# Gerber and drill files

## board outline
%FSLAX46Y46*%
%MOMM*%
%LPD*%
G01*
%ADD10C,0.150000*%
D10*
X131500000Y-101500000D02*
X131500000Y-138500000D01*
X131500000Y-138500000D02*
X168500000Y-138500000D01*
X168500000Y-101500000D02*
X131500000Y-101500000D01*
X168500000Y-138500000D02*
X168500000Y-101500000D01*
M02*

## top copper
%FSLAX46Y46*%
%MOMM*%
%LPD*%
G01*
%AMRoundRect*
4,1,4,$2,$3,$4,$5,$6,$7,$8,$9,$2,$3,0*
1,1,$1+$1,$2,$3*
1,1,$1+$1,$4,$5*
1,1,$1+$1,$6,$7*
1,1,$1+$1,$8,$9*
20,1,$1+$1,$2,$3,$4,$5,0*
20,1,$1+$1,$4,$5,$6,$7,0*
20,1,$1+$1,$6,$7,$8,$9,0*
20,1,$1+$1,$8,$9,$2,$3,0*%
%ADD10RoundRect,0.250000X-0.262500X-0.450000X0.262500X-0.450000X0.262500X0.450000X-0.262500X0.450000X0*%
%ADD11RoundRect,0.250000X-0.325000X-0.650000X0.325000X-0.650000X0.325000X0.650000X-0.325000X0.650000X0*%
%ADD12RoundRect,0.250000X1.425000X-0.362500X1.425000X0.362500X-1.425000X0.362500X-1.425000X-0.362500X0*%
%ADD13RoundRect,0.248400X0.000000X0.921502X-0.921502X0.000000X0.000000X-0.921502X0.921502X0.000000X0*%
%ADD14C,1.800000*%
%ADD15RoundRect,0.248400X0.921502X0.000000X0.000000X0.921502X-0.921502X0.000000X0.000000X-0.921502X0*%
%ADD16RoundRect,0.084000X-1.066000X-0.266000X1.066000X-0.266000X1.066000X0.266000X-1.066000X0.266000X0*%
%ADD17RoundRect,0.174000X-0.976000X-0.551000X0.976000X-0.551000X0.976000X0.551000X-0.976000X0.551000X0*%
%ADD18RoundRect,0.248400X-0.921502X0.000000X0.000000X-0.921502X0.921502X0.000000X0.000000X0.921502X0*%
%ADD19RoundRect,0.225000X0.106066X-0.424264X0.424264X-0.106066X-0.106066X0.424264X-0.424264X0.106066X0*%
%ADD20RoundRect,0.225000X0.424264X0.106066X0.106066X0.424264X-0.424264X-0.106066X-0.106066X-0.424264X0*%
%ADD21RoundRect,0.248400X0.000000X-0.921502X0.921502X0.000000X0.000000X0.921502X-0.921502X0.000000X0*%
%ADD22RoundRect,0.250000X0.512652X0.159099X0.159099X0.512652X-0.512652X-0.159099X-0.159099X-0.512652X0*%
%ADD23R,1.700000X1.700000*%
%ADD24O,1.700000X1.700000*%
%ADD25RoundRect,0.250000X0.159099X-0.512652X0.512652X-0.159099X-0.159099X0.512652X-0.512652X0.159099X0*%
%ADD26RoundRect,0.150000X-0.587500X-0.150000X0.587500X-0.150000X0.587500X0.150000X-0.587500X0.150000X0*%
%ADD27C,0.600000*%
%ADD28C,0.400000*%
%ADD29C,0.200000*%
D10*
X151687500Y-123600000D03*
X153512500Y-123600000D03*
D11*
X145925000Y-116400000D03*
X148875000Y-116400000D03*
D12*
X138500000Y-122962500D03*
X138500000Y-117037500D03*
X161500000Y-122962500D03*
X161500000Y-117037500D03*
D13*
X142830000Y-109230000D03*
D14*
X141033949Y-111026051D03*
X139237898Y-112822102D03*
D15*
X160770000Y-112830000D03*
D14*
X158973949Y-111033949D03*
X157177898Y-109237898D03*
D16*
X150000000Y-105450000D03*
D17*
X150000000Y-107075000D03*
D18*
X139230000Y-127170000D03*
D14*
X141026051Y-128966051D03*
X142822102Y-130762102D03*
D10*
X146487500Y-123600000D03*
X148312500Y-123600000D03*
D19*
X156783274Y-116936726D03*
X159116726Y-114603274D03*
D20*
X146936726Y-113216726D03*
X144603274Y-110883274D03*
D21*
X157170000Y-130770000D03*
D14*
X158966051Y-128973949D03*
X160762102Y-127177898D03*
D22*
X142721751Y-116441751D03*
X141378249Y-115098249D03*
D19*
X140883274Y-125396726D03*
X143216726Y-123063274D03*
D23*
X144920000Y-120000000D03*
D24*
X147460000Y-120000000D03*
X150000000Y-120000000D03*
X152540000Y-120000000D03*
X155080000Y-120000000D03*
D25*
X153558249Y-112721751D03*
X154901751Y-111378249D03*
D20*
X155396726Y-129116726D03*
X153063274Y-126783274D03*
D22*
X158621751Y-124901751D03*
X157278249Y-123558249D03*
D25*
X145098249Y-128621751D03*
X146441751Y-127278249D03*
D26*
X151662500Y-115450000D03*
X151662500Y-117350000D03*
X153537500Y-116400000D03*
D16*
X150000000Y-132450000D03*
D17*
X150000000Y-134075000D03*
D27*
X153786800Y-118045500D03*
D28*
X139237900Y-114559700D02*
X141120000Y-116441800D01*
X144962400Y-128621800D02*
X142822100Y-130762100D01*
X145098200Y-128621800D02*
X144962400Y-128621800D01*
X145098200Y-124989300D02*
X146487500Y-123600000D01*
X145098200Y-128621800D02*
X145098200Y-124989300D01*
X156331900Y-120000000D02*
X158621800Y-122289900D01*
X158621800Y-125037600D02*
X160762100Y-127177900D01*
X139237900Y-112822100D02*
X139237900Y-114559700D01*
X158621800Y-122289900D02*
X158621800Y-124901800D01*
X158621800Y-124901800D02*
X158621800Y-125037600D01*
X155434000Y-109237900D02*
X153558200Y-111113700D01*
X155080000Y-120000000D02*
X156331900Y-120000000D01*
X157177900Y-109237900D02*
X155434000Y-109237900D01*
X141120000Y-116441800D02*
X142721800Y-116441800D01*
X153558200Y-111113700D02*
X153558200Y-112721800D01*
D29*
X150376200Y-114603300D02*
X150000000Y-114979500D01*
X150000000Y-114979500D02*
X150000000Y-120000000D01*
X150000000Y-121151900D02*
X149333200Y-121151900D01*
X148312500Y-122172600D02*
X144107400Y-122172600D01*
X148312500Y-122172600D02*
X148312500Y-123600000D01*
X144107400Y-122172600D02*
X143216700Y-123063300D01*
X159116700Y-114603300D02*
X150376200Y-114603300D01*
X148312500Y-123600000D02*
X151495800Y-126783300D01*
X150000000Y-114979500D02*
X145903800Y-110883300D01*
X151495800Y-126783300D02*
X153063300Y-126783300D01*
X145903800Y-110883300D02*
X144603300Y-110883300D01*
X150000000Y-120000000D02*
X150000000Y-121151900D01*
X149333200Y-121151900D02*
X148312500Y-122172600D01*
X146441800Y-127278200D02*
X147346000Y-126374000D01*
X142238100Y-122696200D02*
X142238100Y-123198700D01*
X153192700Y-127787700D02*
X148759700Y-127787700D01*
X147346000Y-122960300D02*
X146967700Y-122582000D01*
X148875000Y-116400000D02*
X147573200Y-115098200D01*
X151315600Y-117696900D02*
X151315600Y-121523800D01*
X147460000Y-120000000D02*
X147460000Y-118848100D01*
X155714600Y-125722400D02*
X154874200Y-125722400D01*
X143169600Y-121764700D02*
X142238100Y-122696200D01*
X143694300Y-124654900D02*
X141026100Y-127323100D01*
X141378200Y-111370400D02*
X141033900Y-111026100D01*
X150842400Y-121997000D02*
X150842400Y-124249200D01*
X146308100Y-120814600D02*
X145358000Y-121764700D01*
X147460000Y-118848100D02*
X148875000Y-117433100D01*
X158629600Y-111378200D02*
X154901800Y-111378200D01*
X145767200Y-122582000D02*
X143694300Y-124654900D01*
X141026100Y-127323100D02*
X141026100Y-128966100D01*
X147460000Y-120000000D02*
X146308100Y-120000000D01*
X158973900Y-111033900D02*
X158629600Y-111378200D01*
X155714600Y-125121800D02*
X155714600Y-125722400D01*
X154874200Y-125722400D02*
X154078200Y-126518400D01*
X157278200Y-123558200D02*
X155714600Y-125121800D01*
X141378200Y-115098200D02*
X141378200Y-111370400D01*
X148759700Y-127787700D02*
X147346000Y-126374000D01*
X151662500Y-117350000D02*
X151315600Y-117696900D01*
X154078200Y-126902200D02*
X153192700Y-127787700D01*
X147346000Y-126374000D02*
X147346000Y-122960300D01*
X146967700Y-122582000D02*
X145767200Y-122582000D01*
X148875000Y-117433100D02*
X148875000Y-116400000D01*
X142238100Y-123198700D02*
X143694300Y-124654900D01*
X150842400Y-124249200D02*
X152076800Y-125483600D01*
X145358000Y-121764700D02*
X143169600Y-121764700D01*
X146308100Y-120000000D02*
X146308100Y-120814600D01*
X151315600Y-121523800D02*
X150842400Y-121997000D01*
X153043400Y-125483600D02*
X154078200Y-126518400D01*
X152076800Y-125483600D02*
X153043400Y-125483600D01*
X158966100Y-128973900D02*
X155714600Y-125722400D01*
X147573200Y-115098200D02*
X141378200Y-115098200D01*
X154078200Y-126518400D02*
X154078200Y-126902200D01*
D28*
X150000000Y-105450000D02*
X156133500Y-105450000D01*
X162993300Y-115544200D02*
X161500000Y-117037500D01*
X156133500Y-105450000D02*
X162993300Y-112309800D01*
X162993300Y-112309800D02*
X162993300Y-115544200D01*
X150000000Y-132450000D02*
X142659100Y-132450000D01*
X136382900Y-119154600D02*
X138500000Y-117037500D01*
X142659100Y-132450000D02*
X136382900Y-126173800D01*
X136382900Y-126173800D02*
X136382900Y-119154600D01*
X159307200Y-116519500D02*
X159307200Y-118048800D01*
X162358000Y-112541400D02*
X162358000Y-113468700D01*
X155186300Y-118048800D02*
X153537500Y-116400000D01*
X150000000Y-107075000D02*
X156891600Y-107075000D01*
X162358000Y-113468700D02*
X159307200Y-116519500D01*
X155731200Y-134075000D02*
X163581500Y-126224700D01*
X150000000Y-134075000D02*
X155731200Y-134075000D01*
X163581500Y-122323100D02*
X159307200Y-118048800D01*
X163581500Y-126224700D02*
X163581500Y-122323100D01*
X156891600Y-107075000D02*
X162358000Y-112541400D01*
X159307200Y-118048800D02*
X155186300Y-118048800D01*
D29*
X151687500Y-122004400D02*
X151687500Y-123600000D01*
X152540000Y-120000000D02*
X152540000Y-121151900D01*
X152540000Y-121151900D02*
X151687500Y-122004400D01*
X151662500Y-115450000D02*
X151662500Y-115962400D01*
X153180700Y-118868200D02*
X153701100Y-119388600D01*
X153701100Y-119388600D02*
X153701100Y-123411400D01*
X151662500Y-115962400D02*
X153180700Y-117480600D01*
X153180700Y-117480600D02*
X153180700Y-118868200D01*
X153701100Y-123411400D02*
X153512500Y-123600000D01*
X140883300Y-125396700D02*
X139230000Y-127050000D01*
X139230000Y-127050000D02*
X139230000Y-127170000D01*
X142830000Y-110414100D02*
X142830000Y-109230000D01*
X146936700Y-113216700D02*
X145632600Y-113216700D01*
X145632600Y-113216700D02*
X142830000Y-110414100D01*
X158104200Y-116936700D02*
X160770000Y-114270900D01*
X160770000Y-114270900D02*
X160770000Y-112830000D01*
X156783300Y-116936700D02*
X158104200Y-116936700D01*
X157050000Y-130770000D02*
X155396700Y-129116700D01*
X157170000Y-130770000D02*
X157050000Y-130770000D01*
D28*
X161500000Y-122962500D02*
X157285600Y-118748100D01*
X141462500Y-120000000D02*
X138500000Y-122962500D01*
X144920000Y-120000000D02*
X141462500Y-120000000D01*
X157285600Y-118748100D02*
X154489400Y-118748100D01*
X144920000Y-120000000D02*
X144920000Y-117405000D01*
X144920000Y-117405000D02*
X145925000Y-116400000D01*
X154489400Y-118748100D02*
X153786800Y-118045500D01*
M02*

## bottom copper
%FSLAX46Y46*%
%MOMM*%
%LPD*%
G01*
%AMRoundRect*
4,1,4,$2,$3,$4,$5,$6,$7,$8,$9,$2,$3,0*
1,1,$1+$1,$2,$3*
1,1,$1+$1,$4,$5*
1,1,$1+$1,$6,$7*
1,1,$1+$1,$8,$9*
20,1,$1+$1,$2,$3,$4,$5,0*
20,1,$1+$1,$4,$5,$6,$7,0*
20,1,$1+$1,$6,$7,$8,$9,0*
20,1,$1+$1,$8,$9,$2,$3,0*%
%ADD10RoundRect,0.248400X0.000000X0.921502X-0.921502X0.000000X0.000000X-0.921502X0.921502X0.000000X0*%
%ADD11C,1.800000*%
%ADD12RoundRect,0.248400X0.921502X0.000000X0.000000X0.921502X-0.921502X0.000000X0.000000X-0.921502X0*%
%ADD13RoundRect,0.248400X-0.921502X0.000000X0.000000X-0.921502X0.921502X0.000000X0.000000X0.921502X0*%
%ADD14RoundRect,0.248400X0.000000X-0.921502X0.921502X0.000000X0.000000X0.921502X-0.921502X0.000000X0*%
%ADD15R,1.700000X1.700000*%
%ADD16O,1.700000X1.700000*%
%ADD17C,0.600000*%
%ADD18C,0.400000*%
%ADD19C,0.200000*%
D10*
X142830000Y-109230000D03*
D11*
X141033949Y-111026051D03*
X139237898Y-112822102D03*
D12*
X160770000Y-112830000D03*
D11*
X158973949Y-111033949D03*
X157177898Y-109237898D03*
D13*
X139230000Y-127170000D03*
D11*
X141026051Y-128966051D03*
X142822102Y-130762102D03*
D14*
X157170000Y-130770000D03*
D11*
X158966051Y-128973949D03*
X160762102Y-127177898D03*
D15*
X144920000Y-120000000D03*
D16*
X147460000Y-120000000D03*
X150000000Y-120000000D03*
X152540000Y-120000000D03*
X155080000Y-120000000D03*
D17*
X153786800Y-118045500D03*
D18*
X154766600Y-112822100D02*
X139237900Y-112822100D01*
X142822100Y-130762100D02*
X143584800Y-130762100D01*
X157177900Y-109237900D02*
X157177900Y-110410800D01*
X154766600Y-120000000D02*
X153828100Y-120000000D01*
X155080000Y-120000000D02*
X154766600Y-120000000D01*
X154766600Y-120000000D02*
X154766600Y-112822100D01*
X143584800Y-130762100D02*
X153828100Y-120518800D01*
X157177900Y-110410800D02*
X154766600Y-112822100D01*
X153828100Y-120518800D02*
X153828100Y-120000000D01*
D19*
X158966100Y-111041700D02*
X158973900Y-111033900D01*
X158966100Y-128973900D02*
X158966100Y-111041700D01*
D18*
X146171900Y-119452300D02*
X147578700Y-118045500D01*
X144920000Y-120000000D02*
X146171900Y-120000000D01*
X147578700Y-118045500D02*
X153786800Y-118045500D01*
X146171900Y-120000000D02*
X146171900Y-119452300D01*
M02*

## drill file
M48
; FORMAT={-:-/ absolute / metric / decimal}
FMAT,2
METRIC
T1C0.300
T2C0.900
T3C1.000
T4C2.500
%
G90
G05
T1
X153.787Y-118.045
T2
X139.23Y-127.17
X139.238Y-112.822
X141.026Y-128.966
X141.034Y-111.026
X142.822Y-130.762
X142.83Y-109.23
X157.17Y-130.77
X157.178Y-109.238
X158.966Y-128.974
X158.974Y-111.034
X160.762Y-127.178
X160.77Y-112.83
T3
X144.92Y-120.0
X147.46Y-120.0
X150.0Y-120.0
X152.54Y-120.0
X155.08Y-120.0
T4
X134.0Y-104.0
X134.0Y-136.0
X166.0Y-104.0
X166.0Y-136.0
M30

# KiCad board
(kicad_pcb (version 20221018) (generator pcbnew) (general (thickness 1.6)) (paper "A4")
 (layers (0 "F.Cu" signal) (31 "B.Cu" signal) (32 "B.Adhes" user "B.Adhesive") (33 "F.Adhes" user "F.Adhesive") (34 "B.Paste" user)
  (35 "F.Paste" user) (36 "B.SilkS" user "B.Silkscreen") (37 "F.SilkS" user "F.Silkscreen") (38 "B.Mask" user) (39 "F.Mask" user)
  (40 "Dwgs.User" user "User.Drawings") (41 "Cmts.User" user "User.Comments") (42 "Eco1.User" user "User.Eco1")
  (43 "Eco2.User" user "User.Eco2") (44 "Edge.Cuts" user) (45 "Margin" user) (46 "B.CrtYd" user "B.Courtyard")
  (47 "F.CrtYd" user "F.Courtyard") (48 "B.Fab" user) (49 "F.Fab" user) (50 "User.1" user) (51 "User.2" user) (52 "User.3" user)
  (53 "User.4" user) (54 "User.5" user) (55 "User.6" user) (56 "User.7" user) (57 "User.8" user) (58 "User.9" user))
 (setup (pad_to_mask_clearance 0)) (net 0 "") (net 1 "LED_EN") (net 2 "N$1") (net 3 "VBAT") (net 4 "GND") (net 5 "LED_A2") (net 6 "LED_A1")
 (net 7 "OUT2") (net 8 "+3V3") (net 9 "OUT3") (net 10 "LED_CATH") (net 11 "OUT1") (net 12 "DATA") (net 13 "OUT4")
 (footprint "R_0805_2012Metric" (layer "F.Cu") (at 152.6 123.6)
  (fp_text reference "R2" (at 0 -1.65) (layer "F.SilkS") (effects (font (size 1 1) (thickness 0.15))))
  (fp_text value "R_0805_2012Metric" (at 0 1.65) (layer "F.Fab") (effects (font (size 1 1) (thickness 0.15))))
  (pad "1" smd roundrect (at -0.9125 0) (size 1.025 1.4) (layers "F.Cu" "F.Paste" "F.Mask") (roundrect_rratio 0.243902) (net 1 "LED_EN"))
  (pad "2" smd roundrect (at 0.9125 0) (size 1.025 1.4) (layers "F.Cu" "F.Paste" "F.Mask") (roundrect_rratio 0.243902) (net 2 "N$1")))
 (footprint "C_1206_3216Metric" (layer "F.Cu") (at 147.4 116.4)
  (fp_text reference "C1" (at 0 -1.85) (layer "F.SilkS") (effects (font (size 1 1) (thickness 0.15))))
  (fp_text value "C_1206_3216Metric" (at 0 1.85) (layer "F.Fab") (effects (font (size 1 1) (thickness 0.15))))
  (pad "1" smd roundrect (at -1.475 0) (size 1.15 1.8) (layers "F.Cu" "F.Paste" "F.Mask") (roundrect_rratio 0.217391) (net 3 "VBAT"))
  (pad "2" smd roundrect (at 1.475 0) (size 1.15 1.8) (layers "F.Cu" "F.Paste" "F.Mask") (roundrect_rratio 0.217391) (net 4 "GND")))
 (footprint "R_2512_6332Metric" (layer "F.Cu") (at 138.5 120 90)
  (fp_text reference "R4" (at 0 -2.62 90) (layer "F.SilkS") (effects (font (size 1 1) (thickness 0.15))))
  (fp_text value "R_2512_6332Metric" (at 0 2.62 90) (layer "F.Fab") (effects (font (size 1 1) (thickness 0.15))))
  (pad "1" smd roundrect (at -2.9625 0 90) (size 1.225 3.35) (layers "F.Cu" "F.Paste" "F.Mask") (roundrect_rratio 0.204082) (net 3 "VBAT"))
  (pad "2" smd roundrect (at 2.9625 0 90) (size 1.225 3.35) (layers "F.Cu" "F.Paste" "F.Mask") (roundrect_rratio 0.204082) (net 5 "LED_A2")))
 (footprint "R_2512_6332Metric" (layer "F.Cu") (at 161.5 120 90)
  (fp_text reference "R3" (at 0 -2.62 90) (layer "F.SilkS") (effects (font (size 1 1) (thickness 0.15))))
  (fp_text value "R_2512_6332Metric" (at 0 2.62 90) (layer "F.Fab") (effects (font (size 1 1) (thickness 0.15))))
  (pad "1" smd roundrect (at -2.9625 0 90) (size 1.225 3.35) (layers "F.Cu" "F.Paste" "F.Mask") (roundrect_rratio 0.204082) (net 3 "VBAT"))
  (pad "2" smd roundrect (at 2.9625 0 90) (size 1.225 3.35) (layers "F.Cu" "F.Paste" "F.Mask") (roundrect_rratio 0.204082) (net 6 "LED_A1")))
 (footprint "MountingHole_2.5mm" (layer "F.Cu") (at 134 104)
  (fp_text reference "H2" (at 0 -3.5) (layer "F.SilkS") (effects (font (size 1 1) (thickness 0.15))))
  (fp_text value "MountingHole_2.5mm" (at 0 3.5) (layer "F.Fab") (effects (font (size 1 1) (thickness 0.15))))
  (pad "" np_thru_hole circle (at 0 0) (size 2.5 2.5) (drill 2.5) (layers "*.Cu" "*.Mask")))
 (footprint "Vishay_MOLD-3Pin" (layer "F.Cu") (at 142.83 109.23 -135)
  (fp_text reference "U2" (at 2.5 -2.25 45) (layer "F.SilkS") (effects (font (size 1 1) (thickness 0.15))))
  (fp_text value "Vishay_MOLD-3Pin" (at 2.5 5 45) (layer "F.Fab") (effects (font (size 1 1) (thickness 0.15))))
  (pad "1" thru_hole roundrect (at 0 0 225) (size 1.8 1.8) (drill 0.9) (layers "*.Cu" "*.Mask") (roundrect_rratio 0.138) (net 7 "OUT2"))
  (pad "2" thru_hole circle (at 2.54 0 225) (size 1.8 1.8) (drill 0.9) (layers "*.Cu" "*.Mask") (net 4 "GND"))
  (pad "3" thru_hole circle (at 5.08 0 225) (size 1.8 1.8) (drill 0.9) (layers "*.Cu" "*.Mask") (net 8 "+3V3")))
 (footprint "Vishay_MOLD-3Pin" (layer "F.Cu") (at 160.77 112.83 135)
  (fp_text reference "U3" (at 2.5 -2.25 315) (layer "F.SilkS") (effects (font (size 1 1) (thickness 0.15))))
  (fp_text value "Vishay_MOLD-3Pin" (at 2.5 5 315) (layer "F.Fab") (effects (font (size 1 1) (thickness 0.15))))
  (pad "1" thru_hole roundrect (at 0 0 135) (size 1.8 1.8) (drill 0.9) (layers "*.Cu" "*.Mask") (roundrect_rratio 0.138) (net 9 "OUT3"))
  (pad "2" thru_hole circle (at 2.54 0 135) (size 1.8 1.8) (drill 0.9) (layers "*.Cu" "*.Mask") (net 4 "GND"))
  (pad "3" thru_hole circle (at 5.08 0 135) (size 1.8 1.8) (drill 0.9) (layers "*.Cu" "*.Mask") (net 8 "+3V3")))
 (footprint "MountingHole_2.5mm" (layer "F.Cu") (at 166 136)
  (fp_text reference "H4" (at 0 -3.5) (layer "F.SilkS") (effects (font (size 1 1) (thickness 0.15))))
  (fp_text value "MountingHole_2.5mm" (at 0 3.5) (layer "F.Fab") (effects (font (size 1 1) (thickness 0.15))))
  (pad "" np_thru_hole circle (at 0 0) (size 2.5 2.5) (drill 2.5) (layers "*.Cu" "*.Mask")))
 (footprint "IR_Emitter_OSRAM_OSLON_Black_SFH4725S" (layer "F.Cu") (at 150 106.5)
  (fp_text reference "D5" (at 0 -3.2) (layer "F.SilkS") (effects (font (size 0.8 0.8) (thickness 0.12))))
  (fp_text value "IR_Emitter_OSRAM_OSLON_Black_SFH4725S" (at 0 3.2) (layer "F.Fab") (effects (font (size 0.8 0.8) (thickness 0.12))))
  (pad "1" smd roundrect (at 0 -1.05) (size 2.3 0.7) (layers "F.Cu" "F.Paste" "F.Mask") (roundrect_rratio 0.12) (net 6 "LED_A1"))
  (pad "2" smd roundrect (at 0 0.575) (size 2.3 1.45) (layers "F.Cu" "F.Paste" "F.Mask") (roundrect_rratio 0.12) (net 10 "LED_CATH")))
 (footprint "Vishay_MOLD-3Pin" (layer "F.Cu") (at 139.23 127.17 -45)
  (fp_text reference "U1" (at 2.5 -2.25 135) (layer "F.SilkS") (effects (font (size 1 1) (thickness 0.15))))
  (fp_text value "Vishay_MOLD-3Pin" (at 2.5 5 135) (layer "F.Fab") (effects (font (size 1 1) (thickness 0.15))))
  (pad "1" thru_hole roundrect (at 0 0 315) (size 1.8 1.8) (drill 0.9) (layers "*.Cu" "*.Mask") (roundrect_rratio 0.138) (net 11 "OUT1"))
  (pad "2" thru_hole circle (at 2.54 0 315) (size 1.8 1.8) (drill 0.9) (layers "*.Cu" "*.Mask") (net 4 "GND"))
  (pad "3" thru_hole circle (at 5.08 0 315) (size 1.8 1.8) (drill 0.9) (layers "*.Cu" "*.Mask") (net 8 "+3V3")))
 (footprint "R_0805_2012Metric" (layer "F.Cu") (at 147.4 123.6)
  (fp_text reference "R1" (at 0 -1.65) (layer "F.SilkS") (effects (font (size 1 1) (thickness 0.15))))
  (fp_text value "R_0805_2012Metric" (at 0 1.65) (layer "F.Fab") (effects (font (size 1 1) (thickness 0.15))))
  (pad "1" smd roundrect (at -0.9125 0) (size 1.025 1.4) (layers "F.Cu" "F.Paste" "F.Mask") (roundrect_rratio 0.243902) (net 8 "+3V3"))
  (pad "2" smd roundrect (at 0.9125 0) (size 1.025 1.4) (layers "F.Cu" "F.Paste" "F.Mask") (roundrect_rratio 0.243902) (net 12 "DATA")))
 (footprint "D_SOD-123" (layer "F.Cu") (at 157.95 115.77 45)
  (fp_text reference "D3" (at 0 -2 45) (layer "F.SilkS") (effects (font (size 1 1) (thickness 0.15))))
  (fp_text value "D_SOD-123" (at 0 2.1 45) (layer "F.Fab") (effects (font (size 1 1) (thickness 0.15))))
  (pad "1" smd roundrect (at -1.65 0 45) (size 0.9 1.2) (layers "F.Cu" "F.Paste" "F.Mask") (roundrect_rratio 0.25) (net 9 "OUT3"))
  (pad "2" smd roundrect (at 1.65 0 45) (size 0.9 1.2) (layers "F.Cu" "F.Paste" "F.Mask") (roundrect_rratio 0.25) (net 12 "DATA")))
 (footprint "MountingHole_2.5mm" (layer "F.Cu") (at 134 136)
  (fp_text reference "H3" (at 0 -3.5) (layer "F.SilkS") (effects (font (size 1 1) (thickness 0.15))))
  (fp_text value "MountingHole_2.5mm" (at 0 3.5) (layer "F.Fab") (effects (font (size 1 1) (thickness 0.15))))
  (pad "" np_thru_hole circle (at 0 0) (size 2.5 2.5) (drill 2.5) (layers "*.Cu" "*.Mask")))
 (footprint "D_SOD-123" (layer "F.Cu") (at 145.77 112.05 135)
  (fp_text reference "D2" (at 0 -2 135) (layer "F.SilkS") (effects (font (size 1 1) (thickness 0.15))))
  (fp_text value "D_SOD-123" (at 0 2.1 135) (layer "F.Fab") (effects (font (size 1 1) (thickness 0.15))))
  (pad "1" smd roundrect (at -1.65 0 135) (size 0.9 1.2) (layers "F.Cu" "F.Paste" "F.Mask") (roundrect_rratio 0.25) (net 7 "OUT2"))
  (pad "2" smd roundrect (at 1.65 0 135) (size 0.9 1.2) (layers "F.Cu" "F.Paste" "F.Mask") (roundrect_rratio 0.25) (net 12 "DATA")))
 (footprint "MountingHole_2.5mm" (layer "F.Cu") (at 166 104)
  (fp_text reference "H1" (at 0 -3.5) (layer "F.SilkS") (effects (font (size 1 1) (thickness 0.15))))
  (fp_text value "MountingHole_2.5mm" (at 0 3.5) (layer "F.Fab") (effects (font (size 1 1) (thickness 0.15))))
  (pad "" np_thru_hole circle (at 0 0) (size 2.5 2.5) (drill 2.5) (layers "*.Cu" "*.Mask")))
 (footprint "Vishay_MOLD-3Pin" (layer "F.Cu") (at 157.17 130.77 45)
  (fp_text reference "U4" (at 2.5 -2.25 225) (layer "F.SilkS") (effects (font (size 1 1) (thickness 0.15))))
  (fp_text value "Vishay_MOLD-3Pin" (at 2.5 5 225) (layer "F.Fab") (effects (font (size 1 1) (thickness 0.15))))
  (pad "1" thru_hole roundrect (at 0 0 45) (size 1.8 1.8) (drill 0.9) (layers "*.Cu" "*.Mask") (roundrect_rratio 0.138) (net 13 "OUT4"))
  (pad "2" thru_hole circle (at 2.54 0 45) (size 1.8 1.8) (drill 0.9) (layers "*.Cu" "*.Mask") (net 4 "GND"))
  (pad "3" thru_hole circle (at 5.08 0 45) (size 1.8 1.8) (drill 0.9) (layers "*.Cu" "*.Mask") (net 8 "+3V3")))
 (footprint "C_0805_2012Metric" (layer "F.Cu") (at 142.05 115.77 135)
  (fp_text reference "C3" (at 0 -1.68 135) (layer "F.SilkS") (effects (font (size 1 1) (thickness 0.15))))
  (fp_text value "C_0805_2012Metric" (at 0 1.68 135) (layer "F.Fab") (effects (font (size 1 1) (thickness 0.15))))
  (pad "1" smd roundrect (at -0.95 0 135) (size 1 1.45) (layers "F.Cu" "F.Paste" "F.Mask") (roundrect_rratio 0.25) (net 8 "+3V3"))
  (pad "2" smd roundrect (at 0.95 0 135) (size 1 1.45) (layers "F.Cu" "F.Paste" "F.Mask") (roundrect_rratio 0.25) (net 4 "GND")))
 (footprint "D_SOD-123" (layer "F.Cu") (at 142.05 124.23 45)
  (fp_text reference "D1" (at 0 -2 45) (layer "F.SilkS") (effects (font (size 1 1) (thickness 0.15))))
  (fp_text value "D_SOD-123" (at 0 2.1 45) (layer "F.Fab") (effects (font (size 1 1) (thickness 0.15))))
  (pad "1" smd roundrect (at -1.65 0 45) (size 0.9 1.2) (layers "F.Cu" "F.Paste" "F.Mask") (roundrect_rratio 0.25) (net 11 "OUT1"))
  (pad "2" smd roundrect (at 1.65 0 45) (size 0.9 1.2) (layers "F.Cu" "F.Paste" "F.Mask") (roundrect_rratio 0.25) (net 12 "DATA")))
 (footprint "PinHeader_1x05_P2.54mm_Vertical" (layer "F.Cu") (at 144.92 120 90)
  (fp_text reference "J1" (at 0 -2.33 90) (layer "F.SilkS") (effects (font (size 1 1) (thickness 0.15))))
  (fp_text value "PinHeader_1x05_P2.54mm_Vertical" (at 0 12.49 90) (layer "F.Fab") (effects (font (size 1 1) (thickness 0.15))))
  (pad "1" thru_hole rect (at 0 0 90) (size 1.7 1.7) (drill 1) (layers "*.Cu" "*.Mask") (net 3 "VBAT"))
  (pad "2" thru_hole oval (at 0 2.54 90) (size 1.7 1.7) (drill 1) (layers "*.Cu" "*.Mask") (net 4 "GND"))
  (pad "3" thru_hole oval (at 0 5.08 90) (size 1.7 1.7) (drill 1) (layers "*.Cu" "*.Mask") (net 12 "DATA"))
  (pad "4" thru_hole oval (at 0 7.62 90) (size 1.7 1.7) (drill 1) (layers "*.Cu" "*.Mask") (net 1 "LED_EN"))
  (pad "5" thru_hole oval (at 0 10.16 90) (size 1.7 1.7) (drill 1) (layers "*.Cu" "*.Mask") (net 8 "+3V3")))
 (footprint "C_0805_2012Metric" (layer "F.Cu") (at 154.23 112.05 45)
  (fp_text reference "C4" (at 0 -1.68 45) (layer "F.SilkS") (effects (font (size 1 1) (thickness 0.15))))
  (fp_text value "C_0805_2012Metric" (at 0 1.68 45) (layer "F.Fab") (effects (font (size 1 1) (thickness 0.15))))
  (pad "1" smd roundrect (at -0.95 0 45) (size 1 1.45) (layers "F.Cu" "F.Paste" "F.Mask") (roundrect_rratio 0.25) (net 8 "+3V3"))
  (pad "2" smd roundrect (at 0.95 0 45) (size 1 1.45) (layers "F.Cu" "F.Paste" "F.Mask") (roundrect_rratio 0.25) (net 4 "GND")))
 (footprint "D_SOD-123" (layer "F.Cu") (at 154.23 127.95 135)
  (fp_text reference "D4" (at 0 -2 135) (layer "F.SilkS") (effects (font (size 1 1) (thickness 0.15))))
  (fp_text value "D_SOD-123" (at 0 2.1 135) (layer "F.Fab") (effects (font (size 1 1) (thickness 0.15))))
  (pad "1" smd roundrect (at -1.65 0 135) (size 0.9 1.2) (layers "F.Cu" "F.Paste" "F.Mask") (roundrect_rratio 0.25) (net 13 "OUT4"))
  (pad "2" smd roundrect (at 1.65 0 135) (size 0.9 1.2) (layers "F.Cu" "F.Paste" "F.Mask") (roundrect_rratio 0.25) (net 12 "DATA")))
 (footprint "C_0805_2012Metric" (layer "F.Cu") (at 157.95 124.23 135)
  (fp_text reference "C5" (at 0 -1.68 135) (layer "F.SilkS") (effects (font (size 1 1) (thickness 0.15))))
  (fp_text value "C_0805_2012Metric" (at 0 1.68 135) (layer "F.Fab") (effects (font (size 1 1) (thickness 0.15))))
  (pad "1" smd roundrect (at -0.95 0 135) (size 1 1.45) (layers "F.Cu" "F.Paste" "F.Mask") (roundrect_rratio 0.25) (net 8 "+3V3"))
  (pad "2" smd roundrect (at 0.95 0 135) (size 1 1.45) (layers "F.Cu" "F.Paste" "F.Mask") (roundrect_rratio 0.25) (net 4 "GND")))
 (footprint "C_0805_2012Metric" (layer "F.Cu") (at 145.77 127.95 45)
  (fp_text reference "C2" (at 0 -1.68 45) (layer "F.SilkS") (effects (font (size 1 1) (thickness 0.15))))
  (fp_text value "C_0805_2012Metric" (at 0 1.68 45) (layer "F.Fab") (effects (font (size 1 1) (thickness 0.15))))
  (pad "1" smd roundrect (at -0.95 0 45) (size 1 1.45) (layers "F.Cu" "F.Paste" "F.Mask") (roundrect_rratio 0.25) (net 8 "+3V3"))
  (pad "2" smd roundrect (at 0.95 0 45) (size 1 1.45) (layers "F.Cu" "F.Paste" "F.Mask") (roundrect_rratio 0.25) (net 4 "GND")))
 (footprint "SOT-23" (layer "F.Cu") (at 152.6 116.4)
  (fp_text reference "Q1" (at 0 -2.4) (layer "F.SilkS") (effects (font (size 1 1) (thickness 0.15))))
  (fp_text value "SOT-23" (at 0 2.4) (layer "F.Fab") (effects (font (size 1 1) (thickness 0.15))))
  (pad "1" smd roundrect (at -0.9375 -0.95) (size 1.475 0.6) (layers "F.Cu" "F.Paste" "F.Mask") (roundrect_rratio 0.25) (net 2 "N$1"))
  (pad "2" smd roundrect (at -0.9375 0.95) (size 1.475 0.6) (layers "F.Cu" "F.Paste" "F.Mask") (roundrect_rratio 0.25) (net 4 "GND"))
  (pad "3" smd roundrect (at 0.9375 0) (size 1.475 0.6) (layers "F.Cu" "F.Paste" "F.Mask") (roundrect_rratio 0.25) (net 10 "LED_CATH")))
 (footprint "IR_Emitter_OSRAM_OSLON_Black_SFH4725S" (layer "F.Cu") (at 150 133.5)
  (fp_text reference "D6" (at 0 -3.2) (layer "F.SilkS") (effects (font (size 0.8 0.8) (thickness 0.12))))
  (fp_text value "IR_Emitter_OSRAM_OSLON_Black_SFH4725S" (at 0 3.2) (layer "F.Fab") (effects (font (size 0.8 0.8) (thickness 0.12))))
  (pad "1" smd roundrect (at 0 -1.05) (size 2.3 0.7) (layers "F.Cu" "F.Paste" "F.Mask") (roundrect_rratio 0.12) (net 5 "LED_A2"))
  (pad "2" smd roundrect (at 0 0.575) (size 2.3 1.45) (layers "F.Cu" "F.Paste" "F.Mask") (roundrect_rratio 0.12) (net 10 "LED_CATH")))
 (gr_line (start 131.5 101.5) (end 131.5 138.5) (stroke (width 0.15) (type default)) (layer "Edge.Cuts"))
 (gr_line (start 131.5 138.5) (end 168.5 138.5) (stroke (width 0.15) (type default)) (layer "Edge.Cuts"))
 (gr_line (start 168.5 101.5) (end 131.5 101.5) (stroke (width 0.15) (type default)) (layer "Edge.Cuts"))
 (gr_line (start 168.5 138.5) (end 168.5 101.5) (stroke (width 0.15) (type default)) (layer "Edge.Cuts"))
 (segment (start 139.2379 114.5597) (end 141.12 116.4418) (width 0.4) (layer "F.Cu") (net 8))
 (segment (start 144.9624 128.6218) (end 142.8221 130.7621) (width 0.4) (layer "F.Cu") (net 8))
 (segment (start 145.0982 128.6218) (end 144.9624 128.6218) (width 0.4) (layer "F.Cu") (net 8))
 (segment (start 145.0982 124.9893) (end 146.4875 123.6) (width 0.4) (layer "F.Cu") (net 8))
 (segment (start 145.0982 128.6218) (end 145.0982 124.9893) (width 0.4) (layer "F.Cu") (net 8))
 (segment (start 156.3319 120) (end 158.6218 122.2899) (width 0.4) (layer "F.Cu") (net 8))
 (segment (start 158.6218 125.0376) (end 160.7621 127.1779) (width 0.4) (layer "F.Cu") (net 8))
 (segment (start 139.2379 112.8221) (end 139.2379 114.5597) (width 0.4) (layer "F.Cu") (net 8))
 (segment (start 158.6218 122.2899) (end 158.6218 124.9018) (width 0.4) (layer "F.Cu") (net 8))
 (segment (start 158.6218 124.9018) (end 158.6218 125.0376) (width 0.4) (layer "F.Cu") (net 8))
 (segment (start 155.434 109.2379) (end 153.5582 111.1137) (width 0.4) (layer "F.Cu") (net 8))
 (segment (start 155.08 120) (end 156.3319 120) (width 0.4) (layer "F.Cu") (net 8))
 (segment (start 157.1779 109.2379) (end 155.434 109.2379) (width 0.4) (layer "F.Cu") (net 8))
 (segment (start 141.12 116.4418) (end 142.7218 116.4418) (width 0.4) (layer "F.Cu") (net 8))
 (segment (start 153.5582 111.1137) (end 153.5582 112.7218) (width 0.4) (layer "F.Cu") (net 8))
 (segment (start 154.7666 112.8221) (end 139.2379 112.8221) (width 0.4) (layer "B.Cu") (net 8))
 (segment (start 142.8221 130.7621) (end 143.5848 130.7621) (width 0.4) (layer "B.Cu") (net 8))
 (segment (start 157.1779 109.2379) (end 157.1779 110.4108) (width 0.4) (layer "B.Cu") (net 8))
 (segment (start 154.7666 120) (end 153.8281 120) (width 0.4) (layer "B.Cu") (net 8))
 (segment (start 155.08 120) (end 154.7666 120) (width 0.4) (layer "B.Cu") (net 8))
 (segment (start 154.7666 120) (end 154.7666 112.8221) (width 0.4) (layer "B.Cu") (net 8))
 (segment (start 143.5848 130.7621) (end 153.8281 120.5188) (width 0.4) (layer "B.Cu") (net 8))
 (segment (start 157.1779 110.4108) (end 154.7666 112.8221) (width 0.4) (layer "B.Cu") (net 8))
 (segment (start 153.8281 120.5188) (end 153.8281 120) (width 0.4) (layer "B.Cu") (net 8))
 (segment (start 150.3762 114.6033) (end 150 114.9795) (width 0.2) (layer "F.Cu") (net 12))
 (segment (start 150 114.9795) (end 150 120) (width 0.2) (layer "F.Cu") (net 12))
 (segment (start 150 121.1519) (end 149.3332 121.1519) (width 0.2) (layer "F.Cu") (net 12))
 (segment (start 148.3125 122.1726) (end 144.1074 122.1726) (width 0.2) (layer "F.Cu") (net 12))
 (segment (start 148.3125 122.1726) (end 148.3125 123.6) (width 0.2) (layer "F.Cu") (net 12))
 (segment (start 144.1074 122.1726) (end 143.2167 123.0633) (width 0.2) (layer "F.Cu") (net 12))
 (segment (start 159.1167 114.6033) (end 150.3762 114.6033) (width 0.2) (layer "F.Cu") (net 12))
 (segment (start 148.3125 123.6) (end 151.4958 126.7833) (width 0.2) (layer "F.Cu") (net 12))
 (segment (start 150 114.9795) (end 145.9038 110.8833) (width 0.2) (layer "F.Cu") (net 12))
 (segment (start 151.4958 126.7833) (end 153.0633 126.7833) (width 0.2) (layer "F.Cu") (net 12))
 (segment (start 145.9038 110.8833) (end 144.6033 110.8833) (width 0.2) (layer "F.Cu") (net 12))
 (segment (start 150 120) (end 150 121.1519) (width 0.2) (layer "F.Cu") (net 12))
 (segment (start 149.3332 121.1519) (end 148.3125 122.1726) (width 0.2) (layer "F.Cu") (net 12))
 (segment (start 146.4418 127.2782) (end 147.346 126.374) (width 0.2) (layer "F.Cu") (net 4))
 (segment (start 142.2381 122.6962) (end 142.2381 123.1987) (width 0.2) (layer "F.Cu") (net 4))
 (segment (start 153.1927 127.7877) (end 148.7597 127.7877) (width 0.2) (layer "F.Cu") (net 4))
 (segment (start 147.346 122.9603) (end 146.9677 122.582) (width 0.2) (layer "F.Cu") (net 4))
 (segment (start 148.875 116.4) (end 147.5732 115.0982) (width 0.2) (layer "F.Cu") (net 4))
 (segment (start 151.3156 117.6969) (end 151.3156 121.5238) (width 0.2) (layer "F.Cu") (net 4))
 (segment (start 147.46 120) (end 147.46 118.8481) (width 0.2) (layer "F.Cu") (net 4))
 (segment (start 155.7146 125.7224) (end 154.8742 125.7224) (width 0.2) (layer "F.Cu") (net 4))
 (segment (start 143.1696 121.7647) (end 142.2381 122.6962) (width 0.2) (layer "F.Cu") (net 4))
 (segment (start 143.6943 124.6549) (end 141.0261 127.3231) (width 0.2) (layer "F.Cu") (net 4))
 (segment (start 141.3782 111.3704) (end 141.0339 111.0261) (width 0.2) (layer "F.Cu") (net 4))
 (segment (start 150.8424 121.997) (end 150.8424 124.2492) (width 0.2) (layer "F.Cu") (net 4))
 (segment (start 146.3081 120.8146) (end 145.358 121.7647) (width 0.2) (layer "F.Cu") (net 4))
 (segment (start 147.46 118.8481) (end 148.875 117.4331) (width 0.2) (layer "F.Cu") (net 4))
 (segment (start 158.6296 111.3782) (end 154.9018 111.3782) (width 0.2) (layer "F.Cu") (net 4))
 (segment (start 145.7672 122.582) (end 143.6943 124.6549) (width 0.2) (layer "F.Cu") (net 4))
 (segment (start 141.0261 127.3231) (end 141.0261 128.9661) (width 0.2) (layer "F.Cu") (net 4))
 (segment (start 147.46 120) (end 146.3081 120) (width 0.2) (layer "F.Cu") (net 4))
 (segment (start 158.9739 111.0339) (end 158.6296 111.3782) (width 0.2) (layer "F.Cu") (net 4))
 (segment (start 155.7146 125.1218) (end 155.7146 125.7224) (width 0.2) (layer "F.Cu") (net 4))
 (segment (start 154.8742 125.7224) (end 154.0782 126.5184) (width 0.2) (layer "F.Cu") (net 4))
 (segment (start 157.2782 123.5582) (end 155.7146 125.1218) (width 0.2) (layer "F.Cu") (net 4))
 (segment (start 141.3782 115.0982) (end 141.3782 111.3704) (width 0.2) (layer "F.Cu") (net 4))
 (segment (start 148.7597 127.7877) (end 147.346 126.374) (width 0.2) (layer "F.Cu") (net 4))
 (segment (start 151.6625 117.35) (end 151.3156 117.6969) (width 0.2) (layer "F.Cu") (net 4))
 (segment (start 154.0782 126.9022) (end 153.1927 127.7877) (width 0.2) (layer "F.Cu") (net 4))
 (segment (start 147.346 126.374) (end 147.346 122.9603) (width 0.2) (layer "F.Cu") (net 4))
 (segment (start 146.9677 122.582) (end 145.7672 122.582) (width 0.2) (layer "F.Cu") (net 4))
 (segment (start 148.875 117.4331) (end 148.875 116.4) (width 0.2) (layer "F.Cu") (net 4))
 (segment (start 142.2381 123.1987) (end 143.6943 124.6549) (width 0.2) (layer "F.Cu") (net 4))
 (segment (start 150.8424 124.2492) (end 152.0768 125.4836) (width 0.2) (layer "F.Cu") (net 4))
 (segment (start 145.358 121.7647) (end 143.1696 121.7647) (width 0.2) (layer "F.Cu") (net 4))
 (segment (start 146.3081 120) (end 146.3081 120.8146) (width 0.2) (layer "F.Cu") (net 4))
 (segment (start 151.3156 121.5238) (end 150.8424 121.997) (width 0.2) (layer "F.Cu") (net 4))
 (segment (start 153.0434 125.4836) (end 154.0782 126.5184) (width 0.2) (layer "F.Cu") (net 4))
 (segment (start 152.0768 125.4836) (end 153.0434 125.4836) (width 0.2) (layer "F.Cu") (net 4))
 (segment (start 158.9661 128.9739) (end 155.7146 125.7224) (width 0.2) (layer "F.Cu") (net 4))
 (segment (start 147.5732 115.0982) (end 141.3782 115.0982) (width 0.2) (layer "F.Cu") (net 4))
 (segment (start 154.0782 126.5184) (end 154.0782 126.9022) (width 0.2) (layer "F.Cu") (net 4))
 (segment (start 158.9661 111.0417) (end 158.9739 111.0339) (width 0.2) (layer "B.Cu") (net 4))
 (segment (start 158.9661 128.9739) (end 158.9661 111.0417) (width 0.2) (layer "B.Cu") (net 4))
 (segment (start 150 105.45) (end 156.1335 105.45) (width 0.4) (layer "F.Cu") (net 6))
 (segment (start 162.9933 115.5442) (end 161.5 117.0375) (width 0.4) (layer "F.Cu") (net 6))
 (segment (start 156.1335 105.45) (end 162.9933 112.3098) (width 0.4) (layer "F.Cu") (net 6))
 (segment (start 162.9933 112.3098) (end 162.9933 115.5442) (width 0.4) (layer "F.Cu") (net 6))
 (segment (start 150 132.45) (end 142.6591 132.45) (width 0.4) (layer "F.Cu") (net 5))
 (segment (start 136.3829 119.1546) (end 138.5 117.0375) (width 0.4) (layer "F.Cu") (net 5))
 (segment (start 142.6591 132.45) (end 136.3829 126.1738) (width 0.4) (layer "F.Cu") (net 5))
 (segment (start 136.3829 126.1738) (end 136.3829 119.1546) (width 0.4) (layer "F.Cu") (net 5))
 (segment (start 159.3072 116.5195) (end 159.3072 118.0488) (width 0.4) (layer "F.Cu") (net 10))
 (segment (start 162.358 112.5414) (end 162.358 113.4687) (width 0.4) (layer "F.Cu") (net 10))
 (segment (start 155.1863 118.0488) (end 153.5375 116.4) (width 0.4) (layer "F.Cu") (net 10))
 (segment (start 150 107.075) (end 156.8916 107.075) (width 0.4) (layer "F.Cu") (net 10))
 (segment (start 162.358 113.4687) (end 159.3072 116.5195) (width 0.4) (layer "F.Cu") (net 10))
 (segment (start 155.7312 134.075) (end 163.5815 126.2247) (width 0.4) (layer "F.Cu") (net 10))
 (segment (start 150 134.075) (end 155.7312 134.075) (width 0.4) (layer "F.Cu") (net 10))
 (segment (start 163.5815 122.3231) (end 159.3072 118.0488) (width 0.4) (layer "F.Cu") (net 10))
 (segment (start 163.5815 126.2247) (end 163.5815 122.3231) (width 0.4) (layer "F.Cu") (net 10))
 (segment (start 156.8916 107.075) (end 162.358 112.5414) (width 0.4) (layer "F.Cu") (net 10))
 (segment (start 159.3072 118.0488) (end 155.1863 118.0488) (width 0.4) (layer "F.Cu") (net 10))
 (segment (start 151.6875 122.0044) (end 151.6875 123.6) (width 0.2) (layer "F.Cu") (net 1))
 (segment (start 152.54 120) (end 152.54 121.1519) (width 0.2) (layer "F.Cu") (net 1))
 (segment (start 152.54 121.1519) (end 151.6875 122.0044) (width 0.2) (layer "F.Cu") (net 1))
 (segment (start 151.6625 115.45) (end 151.6625 115.9624) (width 0.2) (layer "F.Cu") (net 2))
 (segment (start 153.1807 118.8682) (end 153.7011 119.3886) (width 0.2) (layer "F.Cu") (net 2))
 (segment (start 153.7011 119.3886) (end 153.7011 123.4114) (width 0.2) (layer "F.Cu") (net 2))
 (segment (start 151.6625 115.9624) (end 153.1807 117.4806) (width 0.2) (layer "F.Cu") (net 2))
 (segment (start 153.1807 117.4806) (end 153.1807 118.8682) (width 0.2) (layer "F.Cu") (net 2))
 (segment (start 153.7011 123.4114) (end 153.5125 123.6) (width 0.2) (layer "F.Cu") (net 2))
 (segment (start 140.8833 125.3967) (end 139.23 127.05) (width 0.2) (layer "F.Cu") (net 11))
 (segment (start 139.23 127.05) (end 139.23 127.17) (width 0.2) (layer "F.Cu") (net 11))
 (segment (start 142.83 110.4141) (end 142.83 109.23) (width 0.2) (layer "F.Cu") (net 7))
 (segment (start 146.9367 113.2167) (end 145.6326 113.2167) (width 0.2) (layer "F.Cu") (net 7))
 (segment (start 145.6326 113.2167) (end 142.83 110.4141) (width 0.2) (layer "F.Cu") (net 7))
 (segment (start 158.1042 116.9367) (end 160.77 114.2709) (width 0.2) (layer "F.Cu") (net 9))
 (segment (start 160.77 114.2709) (end 160.77 112.83) (width 0.2) (layer "F.Cu") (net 9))
 (segment (start 156.7833 116.9367) (end 158.1042 116.9367) (width 0.2) (layer "F.Cu") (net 9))
 (segment (start 157.05 130.77) (end 155.3967 129.1167) (width 0.2) (layer "F.Cu") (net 13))
 (segment (start 157.17 130.77) (end 157.05 130.77) (width 0.2) (layer "F.Cu") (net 13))
 (segment (start 161.5 122.9625) (end 157.2856 118.7481) (width 0.4) (layer "F.Cu") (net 3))
 (segment (start 141.4625 120) (end 138.5 122.9625) (width 0.4) (layer "F.Cu") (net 3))
 (segment (start 144.92 120) (end 141.4625 120) (width 0.4) (layer "F.Cu") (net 3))
 (segment (start 157.2856 118.7481) (end 154.4894 118.7481) (width 0.4) (layer "F.Cu") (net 3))
 (segment (start 144.92 120) (end 144.92 117.405) (width 0.4) (layer "F.Cu") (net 3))
 (segment (start 144.92 117.405) (end 145.925 116.4) (width 0.4) (layer "F.Cu") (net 3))
 (segment (start 154.4894 118.7481) (end 153.7868 118.0455) (width 0.4) (layer "F.Cu") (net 3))
 (via (at 153.7868 118.0455) (size 0.6) (drill 0.3) (layers "F.Cu" "B.Cu") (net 3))
 (segment (start 146.1719 119.4523) (end 147.5787 118.0455) (width 0.4) (layer "B.Cu") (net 3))
 (segment (start 144.92 120) (end 146.1719 120) (width 0.4) (layer "B.Cu") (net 3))
 (segment (start 147.5787 118.0455) (end 153.7868 118.0455) (width 0.4) (layer "B.Cu") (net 3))
 (segment (start 146.1719 120) (end 146.1719 119.4523) (width 0.4) (layer "B.Cu") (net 3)))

